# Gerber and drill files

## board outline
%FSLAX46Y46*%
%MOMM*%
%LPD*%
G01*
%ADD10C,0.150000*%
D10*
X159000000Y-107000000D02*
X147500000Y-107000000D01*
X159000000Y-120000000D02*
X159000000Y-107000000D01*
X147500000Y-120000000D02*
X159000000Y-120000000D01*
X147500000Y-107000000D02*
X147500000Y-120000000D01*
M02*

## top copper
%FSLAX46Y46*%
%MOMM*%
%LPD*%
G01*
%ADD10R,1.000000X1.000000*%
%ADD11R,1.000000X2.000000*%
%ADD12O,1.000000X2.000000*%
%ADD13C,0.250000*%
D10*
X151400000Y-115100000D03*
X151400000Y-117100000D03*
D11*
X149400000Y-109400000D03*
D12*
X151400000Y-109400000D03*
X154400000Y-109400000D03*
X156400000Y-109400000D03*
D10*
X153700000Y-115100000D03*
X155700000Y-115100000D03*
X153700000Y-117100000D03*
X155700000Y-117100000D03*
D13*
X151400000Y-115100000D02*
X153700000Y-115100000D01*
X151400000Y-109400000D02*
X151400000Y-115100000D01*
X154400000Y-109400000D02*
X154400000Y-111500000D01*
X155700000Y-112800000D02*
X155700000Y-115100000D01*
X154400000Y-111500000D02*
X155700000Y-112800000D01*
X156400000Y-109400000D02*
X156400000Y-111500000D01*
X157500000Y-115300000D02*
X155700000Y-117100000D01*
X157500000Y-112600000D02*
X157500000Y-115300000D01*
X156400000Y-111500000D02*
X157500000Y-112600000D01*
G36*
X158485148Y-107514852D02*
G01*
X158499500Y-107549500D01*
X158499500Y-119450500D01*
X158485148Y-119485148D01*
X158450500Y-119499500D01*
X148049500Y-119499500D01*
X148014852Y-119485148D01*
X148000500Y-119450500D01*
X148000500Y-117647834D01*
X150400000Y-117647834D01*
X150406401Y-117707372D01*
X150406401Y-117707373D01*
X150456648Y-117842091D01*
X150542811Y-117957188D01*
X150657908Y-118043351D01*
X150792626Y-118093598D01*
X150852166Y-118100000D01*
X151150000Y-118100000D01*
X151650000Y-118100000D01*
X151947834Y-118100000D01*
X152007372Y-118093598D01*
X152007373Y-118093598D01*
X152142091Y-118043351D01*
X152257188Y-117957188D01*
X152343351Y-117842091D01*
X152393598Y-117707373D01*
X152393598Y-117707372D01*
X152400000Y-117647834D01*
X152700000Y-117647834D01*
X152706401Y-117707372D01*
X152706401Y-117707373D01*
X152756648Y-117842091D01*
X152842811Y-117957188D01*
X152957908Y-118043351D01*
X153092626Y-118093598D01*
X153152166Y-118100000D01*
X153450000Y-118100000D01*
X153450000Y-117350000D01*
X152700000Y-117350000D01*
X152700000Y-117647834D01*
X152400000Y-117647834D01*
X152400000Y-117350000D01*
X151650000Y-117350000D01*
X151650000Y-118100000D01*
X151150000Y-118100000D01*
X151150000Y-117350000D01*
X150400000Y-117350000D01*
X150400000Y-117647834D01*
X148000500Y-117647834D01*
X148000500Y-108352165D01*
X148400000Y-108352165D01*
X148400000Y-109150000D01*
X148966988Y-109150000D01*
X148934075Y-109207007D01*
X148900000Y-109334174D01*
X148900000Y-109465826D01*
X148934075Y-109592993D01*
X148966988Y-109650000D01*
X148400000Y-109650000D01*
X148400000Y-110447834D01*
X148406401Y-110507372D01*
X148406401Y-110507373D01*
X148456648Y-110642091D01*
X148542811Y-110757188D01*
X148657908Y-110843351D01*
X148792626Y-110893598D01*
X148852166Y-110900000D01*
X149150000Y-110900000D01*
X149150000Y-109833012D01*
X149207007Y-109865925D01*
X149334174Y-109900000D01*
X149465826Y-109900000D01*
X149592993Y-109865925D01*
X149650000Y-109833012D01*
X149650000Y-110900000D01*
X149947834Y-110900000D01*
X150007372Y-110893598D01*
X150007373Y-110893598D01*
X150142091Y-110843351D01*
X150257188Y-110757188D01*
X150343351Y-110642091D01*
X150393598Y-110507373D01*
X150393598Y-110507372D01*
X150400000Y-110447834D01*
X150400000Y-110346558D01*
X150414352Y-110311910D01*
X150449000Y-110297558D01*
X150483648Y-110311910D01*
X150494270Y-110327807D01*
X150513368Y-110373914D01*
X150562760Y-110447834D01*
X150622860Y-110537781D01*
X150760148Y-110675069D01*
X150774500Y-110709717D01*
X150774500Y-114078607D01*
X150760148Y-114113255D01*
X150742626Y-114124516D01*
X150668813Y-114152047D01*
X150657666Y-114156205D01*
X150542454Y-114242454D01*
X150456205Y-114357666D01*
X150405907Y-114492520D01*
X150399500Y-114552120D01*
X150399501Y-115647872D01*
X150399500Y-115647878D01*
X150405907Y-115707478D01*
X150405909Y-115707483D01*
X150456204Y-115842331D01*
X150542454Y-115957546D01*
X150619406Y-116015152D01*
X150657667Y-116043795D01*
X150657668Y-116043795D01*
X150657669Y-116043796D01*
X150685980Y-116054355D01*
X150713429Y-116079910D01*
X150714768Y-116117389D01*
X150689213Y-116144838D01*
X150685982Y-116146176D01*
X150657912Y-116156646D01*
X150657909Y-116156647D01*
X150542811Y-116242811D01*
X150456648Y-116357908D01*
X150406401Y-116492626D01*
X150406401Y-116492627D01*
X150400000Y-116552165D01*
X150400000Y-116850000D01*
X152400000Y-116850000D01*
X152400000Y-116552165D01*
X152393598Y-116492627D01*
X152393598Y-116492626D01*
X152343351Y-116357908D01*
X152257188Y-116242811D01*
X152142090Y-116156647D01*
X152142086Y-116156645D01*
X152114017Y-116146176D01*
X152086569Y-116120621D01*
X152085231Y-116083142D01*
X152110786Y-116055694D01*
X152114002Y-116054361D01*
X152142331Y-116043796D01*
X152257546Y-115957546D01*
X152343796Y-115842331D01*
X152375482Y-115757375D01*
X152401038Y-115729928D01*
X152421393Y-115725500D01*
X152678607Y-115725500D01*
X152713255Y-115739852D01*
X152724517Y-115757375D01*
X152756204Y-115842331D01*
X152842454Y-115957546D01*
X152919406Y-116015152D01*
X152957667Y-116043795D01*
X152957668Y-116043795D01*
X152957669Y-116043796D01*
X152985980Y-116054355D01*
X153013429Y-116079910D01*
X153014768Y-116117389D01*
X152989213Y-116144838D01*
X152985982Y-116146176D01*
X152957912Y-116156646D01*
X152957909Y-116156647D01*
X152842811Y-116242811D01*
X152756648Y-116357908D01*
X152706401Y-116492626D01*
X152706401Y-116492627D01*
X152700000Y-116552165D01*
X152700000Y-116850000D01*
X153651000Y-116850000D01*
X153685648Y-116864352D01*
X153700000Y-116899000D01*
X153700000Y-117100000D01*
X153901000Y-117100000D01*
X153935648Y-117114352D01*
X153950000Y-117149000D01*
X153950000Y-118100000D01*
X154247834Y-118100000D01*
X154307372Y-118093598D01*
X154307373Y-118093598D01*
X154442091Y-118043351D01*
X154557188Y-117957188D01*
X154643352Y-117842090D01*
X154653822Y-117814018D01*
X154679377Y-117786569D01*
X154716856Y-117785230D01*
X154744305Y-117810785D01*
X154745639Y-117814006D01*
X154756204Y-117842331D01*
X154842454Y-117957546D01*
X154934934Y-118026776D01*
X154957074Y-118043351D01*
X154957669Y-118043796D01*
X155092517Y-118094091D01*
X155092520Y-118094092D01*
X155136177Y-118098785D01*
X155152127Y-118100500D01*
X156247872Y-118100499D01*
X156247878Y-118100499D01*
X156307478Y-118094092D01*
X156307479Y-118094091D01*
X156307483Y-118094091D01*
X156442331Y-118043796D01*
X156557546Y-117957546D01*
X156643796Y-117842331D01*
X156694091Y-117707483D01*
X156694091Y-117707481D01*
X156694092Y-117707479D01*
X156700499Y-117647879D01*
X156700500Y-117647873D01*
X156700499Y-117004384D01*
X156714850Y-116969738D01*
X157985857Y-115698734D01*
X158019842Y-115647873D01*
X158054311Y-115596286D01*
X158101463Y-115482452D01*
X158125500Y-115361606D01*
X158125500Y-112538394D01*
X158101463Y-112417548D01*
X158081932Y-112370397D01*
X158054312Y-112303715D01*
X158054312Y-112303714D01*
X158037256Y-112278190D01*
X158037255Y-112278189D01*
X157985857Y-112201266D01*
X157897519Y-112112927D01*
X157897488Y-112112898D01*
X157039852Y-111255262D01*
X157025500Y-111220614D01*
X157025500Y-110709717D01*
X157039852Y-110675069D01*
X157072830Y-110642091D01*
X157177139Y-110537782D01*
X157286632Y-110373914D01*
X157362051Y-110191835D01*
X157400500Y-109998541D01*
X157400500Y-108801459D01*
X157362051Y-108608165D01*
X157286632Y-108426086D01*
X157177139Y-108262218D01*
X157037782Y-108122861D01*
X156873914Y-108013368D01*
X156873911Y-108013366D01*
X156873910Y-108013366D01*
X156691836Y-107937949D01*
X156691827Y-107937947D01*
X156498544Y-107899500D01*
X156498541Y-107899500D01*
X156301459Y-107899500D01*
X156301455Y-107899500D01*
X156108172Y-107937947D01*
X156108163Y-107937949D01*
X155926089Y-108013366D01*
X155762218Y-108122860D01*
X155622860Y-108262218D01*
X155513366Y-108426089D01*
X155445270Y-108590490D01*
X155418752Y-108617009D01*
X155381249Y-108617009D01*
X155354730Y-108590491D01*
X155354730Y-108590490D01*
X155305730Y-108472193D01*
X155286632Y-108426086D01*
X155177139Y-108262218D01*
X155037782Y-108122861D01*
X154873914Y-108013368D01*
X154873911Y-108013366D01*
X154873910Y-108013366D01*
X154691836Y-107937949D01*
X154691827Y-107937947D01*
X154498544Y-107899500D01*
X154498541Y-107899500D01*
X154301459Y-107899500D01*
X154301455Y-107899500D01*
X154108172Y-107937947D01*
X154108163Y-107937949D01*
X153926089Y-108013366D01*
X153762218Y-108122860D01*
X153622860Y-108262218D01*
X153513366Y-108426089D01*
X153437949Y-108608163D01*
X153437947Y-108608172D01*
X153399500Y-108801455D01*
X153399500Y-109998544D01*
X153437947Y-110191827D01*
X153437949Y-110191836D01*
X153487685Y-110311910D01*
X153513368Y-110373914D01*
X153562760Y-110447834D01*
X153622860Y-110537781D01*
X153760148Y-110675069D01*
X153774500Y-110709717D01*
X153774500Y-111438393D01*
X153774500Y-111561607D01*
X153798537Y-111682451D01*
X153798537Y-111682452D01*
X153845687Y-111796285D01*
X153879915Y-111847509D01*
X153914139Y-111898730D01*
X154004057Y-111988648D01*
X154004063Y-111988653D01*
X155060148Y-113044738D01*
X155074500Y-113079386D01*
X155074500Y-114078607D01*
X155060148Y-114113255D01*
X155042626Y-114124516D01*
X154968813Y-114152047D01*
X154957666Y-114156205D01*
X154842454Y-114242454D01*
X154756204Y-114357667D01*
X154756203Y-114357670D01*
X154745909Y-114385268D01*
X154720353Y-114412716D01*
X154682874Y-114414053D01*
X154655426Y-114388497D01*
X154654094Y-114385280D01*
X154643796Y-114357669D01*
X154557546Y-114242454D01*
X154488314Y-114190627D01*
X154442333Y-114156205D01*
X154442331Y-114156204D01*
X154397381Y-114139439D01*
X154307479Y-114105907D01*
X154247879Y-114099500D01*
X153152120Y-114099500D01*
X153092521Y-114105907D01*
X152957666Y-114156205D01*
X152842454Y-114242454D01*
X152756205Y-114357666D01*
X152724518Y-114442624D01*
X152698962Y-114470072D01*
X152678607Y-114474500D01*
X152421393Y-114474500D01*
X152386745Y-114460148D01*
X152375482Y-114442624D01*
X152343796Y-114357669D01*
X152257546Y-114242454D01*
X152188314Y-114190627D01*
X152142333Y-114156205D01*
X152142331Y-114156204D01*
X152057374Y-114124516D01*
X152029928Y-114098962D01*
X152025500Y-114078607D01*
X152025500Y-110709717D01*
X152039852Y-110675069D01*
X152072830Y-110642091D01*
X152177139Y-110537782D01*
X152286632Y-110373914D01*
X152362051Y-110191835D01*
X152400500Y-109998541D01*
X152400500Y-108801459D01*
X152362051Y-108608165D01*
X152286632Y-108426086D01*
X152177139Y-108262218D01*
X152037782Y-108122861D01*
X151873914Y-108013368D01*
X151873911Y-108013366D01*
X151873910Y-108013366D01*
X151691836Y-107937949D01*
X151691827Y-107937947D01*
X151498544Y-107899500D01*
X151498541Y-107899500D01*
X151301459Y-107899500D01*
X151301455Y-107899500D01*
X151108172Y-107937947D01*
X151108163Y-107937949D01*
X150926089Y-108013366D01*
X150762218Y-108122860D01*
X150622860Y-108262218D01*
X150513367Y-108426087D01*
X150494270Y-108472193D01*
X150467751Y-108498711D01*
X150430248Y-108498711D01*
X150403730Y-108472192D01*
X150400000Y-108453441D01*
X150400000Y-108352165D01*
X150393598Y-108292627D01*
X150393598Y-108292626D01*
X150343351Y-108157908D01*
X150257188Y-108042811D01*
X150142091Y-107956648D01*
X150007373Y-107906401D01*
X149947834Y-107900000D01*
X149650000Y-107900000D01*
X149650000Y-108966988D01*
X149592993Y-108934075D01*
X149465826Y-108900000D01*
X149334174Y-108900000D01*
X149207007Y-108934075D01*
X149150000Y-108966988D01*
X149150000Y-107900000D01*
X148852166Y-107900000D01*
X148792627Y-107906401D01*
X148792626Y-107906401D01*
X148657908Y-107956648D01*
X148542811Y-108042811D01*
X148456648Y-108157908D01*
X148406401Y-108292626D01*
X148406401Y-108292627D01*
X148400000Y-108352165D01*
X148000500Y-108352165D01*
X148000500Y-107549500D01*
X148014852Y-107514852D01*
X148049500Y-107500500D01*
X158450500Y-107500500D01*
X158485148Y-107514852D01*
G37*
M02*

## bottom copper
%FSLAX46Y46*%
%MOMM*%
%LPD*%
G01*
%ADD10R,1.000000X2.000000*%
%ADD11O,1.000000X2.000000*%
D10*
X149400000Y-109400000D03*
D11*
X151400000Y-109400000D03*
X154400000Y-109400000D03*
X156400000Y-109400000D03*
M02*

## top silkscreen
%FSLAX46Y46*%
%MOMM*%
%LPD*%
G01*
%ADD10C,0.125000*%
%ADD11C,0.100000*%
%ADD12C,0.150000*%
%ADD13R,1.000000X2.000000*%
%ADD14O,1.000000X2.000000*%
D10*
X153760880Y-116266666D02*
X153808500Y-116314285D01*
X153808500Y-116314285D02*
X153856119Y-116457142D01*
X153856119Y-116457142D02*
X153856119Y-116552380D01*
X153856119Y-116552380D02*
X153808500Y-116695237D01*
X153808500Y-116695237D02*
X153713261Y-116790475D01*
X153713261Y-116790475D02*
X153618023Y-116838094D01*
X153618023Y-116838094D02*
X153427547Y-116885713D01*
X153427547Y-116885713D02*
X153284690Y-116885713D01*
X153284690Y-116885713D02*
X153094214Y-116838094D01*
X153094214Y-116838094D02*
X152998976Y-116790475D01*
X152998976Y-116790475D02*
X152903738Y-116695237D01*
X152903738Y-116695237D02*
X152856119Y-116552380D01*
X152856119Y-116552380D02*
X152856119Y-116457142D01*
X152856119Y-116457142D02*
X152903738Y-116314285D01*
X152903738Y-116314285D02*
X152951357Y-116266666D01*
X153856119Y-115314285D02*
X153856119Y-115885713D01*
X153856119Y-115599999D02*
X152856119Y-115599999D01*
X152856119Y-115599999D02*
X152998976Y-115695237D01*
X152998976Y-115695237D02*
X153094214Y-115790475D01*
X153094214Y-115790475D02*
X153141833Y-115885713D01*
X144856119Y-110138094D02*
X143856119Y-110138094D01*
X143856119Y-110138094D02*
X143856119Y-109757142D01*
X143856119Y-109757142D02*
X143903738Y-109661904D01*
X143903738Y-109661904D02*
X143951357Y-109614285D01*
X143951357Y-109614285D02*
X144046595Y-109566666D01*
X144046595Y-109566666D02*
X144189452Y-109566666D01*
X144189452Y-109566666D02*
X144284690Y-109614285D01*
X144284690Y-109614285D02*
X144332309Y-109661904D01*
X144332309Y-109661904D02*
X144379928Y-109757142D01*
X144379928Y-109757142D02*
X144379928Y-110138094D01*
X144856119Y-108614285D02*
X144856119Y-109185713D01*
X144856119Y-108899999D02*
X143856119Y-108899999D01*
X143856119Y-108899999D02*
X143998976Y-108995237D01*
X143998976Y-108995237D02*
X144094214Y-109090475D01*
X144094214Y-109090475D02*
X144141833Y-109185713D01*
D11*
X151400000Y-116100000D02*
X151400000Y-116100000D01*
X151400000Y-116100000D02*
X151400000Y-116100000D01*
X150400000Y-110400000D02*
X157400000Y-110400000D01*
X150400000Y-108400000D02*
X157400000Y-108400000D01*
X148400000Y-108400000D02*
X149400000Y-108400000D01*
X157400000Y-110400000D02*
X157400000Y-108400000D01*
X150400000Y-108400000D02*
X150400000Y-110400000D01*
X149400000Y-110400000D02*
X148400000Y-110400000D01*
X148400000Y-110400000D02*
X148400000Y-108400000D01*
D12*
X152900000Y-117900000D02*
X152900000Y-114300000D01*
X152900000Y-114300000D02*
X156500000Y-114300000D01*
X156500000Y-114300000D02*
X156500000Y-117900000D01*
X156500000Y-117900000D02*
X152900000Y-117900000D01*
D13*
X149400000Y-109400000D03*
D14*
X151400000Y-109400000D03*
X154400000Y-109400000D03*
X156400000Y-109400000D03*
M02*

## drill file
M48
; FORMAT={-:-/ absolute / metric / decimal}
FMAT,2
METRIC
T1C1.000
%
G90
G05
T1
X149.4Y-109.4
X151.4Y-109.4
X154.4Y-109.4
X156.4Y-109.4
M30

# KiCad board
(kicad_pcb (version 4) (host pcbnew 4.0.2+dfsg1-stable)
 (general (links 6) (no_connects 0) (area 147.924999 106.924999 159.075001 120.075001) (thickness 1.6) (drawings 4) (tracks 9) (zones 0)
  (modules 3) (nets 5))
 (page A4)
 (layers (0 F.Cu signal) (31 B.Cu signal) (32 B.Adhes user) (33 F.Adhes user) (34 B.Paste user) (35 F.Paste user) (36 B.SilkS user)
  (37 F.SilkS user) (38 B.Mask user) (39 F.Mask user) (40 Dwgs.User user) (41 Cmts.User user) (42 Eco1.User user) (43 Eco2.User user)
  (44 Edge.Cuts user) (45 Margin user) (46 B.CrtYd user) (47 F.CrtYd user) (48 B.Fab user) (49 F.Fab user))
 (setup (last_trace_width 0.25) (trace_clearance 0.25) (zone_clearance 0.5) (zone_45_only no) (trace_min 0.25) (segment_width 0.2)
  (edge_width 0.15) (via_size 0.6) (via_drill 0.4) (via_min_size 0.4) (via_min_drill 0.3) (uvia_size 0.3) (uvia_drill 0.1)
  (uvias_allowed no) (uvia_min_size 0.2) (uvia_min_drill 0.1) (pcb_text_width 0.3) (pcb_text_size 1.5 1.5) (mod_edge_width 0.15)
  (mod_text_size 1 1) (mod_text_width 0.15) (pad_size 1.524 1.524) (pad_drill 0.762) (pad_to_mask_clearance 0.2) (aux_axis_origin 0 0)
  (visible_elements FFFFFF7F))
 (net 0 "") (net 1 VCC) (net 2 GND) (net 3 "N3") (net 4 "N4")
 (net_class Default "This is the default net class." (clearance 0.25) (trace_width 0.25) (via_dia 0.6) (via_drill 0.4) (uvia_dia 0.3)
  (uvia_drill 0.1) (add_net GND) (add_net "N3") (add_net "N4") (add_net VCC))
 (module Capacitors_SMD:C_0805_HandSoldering (layer F.Cu) (at 151.4 116.1 270)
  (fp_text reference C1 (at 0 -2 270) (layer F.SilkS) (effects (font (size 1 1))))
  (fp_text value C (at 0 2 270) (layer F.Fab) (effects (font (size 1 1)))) (fp_line (start 0 0) (end 0 0) (layer F.SilkS) (width 0))
  (fp_line (start 0 0) (end 0 0) (layer F.SilkS) (width 0))
  (pad 1 smd rect (at -1 0 270) (size 1 1) (layers F.Cu F.Paste F.Mask) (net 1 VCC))
  (pad 2 smd rect (at 1 0 270) (size 1 1) (layers F.Cu F.Paste F.Mask) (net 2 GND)))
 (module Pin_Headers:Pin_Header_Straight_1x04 (layer F.Cu) (at 149.4 109.4 90)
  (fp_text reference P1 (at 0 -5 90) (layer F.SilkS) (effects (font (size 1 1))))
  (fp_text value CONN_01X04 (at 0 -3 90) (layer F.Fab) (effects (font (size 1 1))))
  (fp_line (start -1 1) (end -1 8) (layer F.SilkS) (width 0)) (fp_line (start 1 1) (end 1 8) (layer F.SilkS) (width 0))
  (fp_line (start 1 -1) (end 1 0) (layer F.SilkS) (width 0)) (fp_line (start -1 8) (end 1 8) (layer F.SilkS) (width 0))
  (fp_line (start 1 1) (end -1 1) (layer F.SilkS) (width 0)) (fp_line (start -1 0) (end -1 -1) (layer F.SilkS) (width 0))
  (fp_line (start -1 -1) (end 1 -1) (layer F.SilkS) (width 0))
  (pad 1 thru_hole rect (at 0 0 90) (size 2 1) (drill 1) (layers *.Cu *.Mask F.SilkS) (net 2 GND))
  (pad 2 thru_hole oval (at 0 2 90) (size 2 1) (drill 1) (layers *.Cu *.Mask F.SilkS) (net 1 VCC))
  (pad 3 thru_hole oval (at 0 5 90) (size 2 1) (drill 1) (layers *.Cu *.Mask F.SilkS) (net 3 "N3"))
  (pad 4 thru_hole oval (at 0 7 90) (size 2 1) (drill 1) (layers *.Cu *.Mask F.SilkS) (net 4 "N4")))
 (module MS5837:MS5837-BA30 (layer F.Cu) (at 154.7 116.1)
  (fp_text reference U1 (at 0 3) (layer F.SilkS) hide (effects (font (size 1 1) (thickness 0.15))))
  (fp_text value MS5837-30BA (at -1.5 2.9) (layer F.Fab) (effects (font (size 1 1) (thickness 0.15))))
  (fp_line (start -1.8 1.8) (end -1.8 -1.8) (layer F.SilkS) (width 0.15))
  (fp_line (start -1.8 -1.8) (end 1.8 -1.8) (layer F.SilkS) (width 0.15))
  (fp_line (start 1.8 -1.8) (end 1.8 1.8) (layer F.SilkS) (width 0.15))
  (fp_line (start 1.8 1.8) (end -1.8 1.8) (layer F.SilkS) (width 0.15))
  (pad 2 smd rect (at -1 -1) (size 1 1) (layers F.Cu F.Paste F.Mask) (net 1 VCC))
  (pad 3 smd rect (at 1 -1) (size 1 1) (layers F.Cu F.Paste F.Mask) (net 3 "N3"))
  (pad 1 smd rect (at -1 1) (size 1 1) (layers F.Cu F.Paste F.Mask) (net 2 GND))
  (pad 4 smd rect (at 1 1) (size 1 1) (layers F.Cu F.Paste F.Mask) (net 4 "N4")))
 (gr_line (start 159 107) (end 147.5 107) (angle 90) (layer Edge.Cuts) (width 0.15))
 (gr_line (start 159 120) (end 159 107) (angle 90) (layer Edge.Cuts) (width 0.15))
 (gr_line (start 147.5 120) (end 159 120) (angle 90) (layer Edge.Cuts) (width 0.15))
 (gr_line (start 147.5 107) (end 147.5 120) (angle 90) (layer Edge.Cuts) (width 0.15))
 (segment (start 151.4 115.1) (end 153.7 115.1) (width 0.25) (layer F.Cu) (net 1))
 (segment (start 151.4 109.4) (end 151.4 115.1) (width 0.25) (layer F.Cu) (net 1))
 (segment (start 154.4 109.4) (end 154.4 111.5) (width 0.25) (layer F.Cu) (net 3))
 (segment (start 155.7 112.8) (end 155.7 115.1) (width 0.25) (layer F.Cu) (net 3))
 (segment (start 154.4 111.5) (end 155.7 112.8) (width 0.25) (layer F.Cu) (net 3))
 (segment (start 156.4 109.4) (end 156.4 111.5) (width 0.25) (layer F.Cu) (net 4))
 (segment (start 157.5 115.3) (end 155.7 117.1) (width 0.25) (layer F.Cu) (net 4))
 (segment (start 157.5 112.6) (end 157.5 115.3) (width 0.25) (layer F.Cu) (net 4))
 (segment (start 156.4 111.5) (end 157.5 112.6) (width 0.25) (layer F.Cu) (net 4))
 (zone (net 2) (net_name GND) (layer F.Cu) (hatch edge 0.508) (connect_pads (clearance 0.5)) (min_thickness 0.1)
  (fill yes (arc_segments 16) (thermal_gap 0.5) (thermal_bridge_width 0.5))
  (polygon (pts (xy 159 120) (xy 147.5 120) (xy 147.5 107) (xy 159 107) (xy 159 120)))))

